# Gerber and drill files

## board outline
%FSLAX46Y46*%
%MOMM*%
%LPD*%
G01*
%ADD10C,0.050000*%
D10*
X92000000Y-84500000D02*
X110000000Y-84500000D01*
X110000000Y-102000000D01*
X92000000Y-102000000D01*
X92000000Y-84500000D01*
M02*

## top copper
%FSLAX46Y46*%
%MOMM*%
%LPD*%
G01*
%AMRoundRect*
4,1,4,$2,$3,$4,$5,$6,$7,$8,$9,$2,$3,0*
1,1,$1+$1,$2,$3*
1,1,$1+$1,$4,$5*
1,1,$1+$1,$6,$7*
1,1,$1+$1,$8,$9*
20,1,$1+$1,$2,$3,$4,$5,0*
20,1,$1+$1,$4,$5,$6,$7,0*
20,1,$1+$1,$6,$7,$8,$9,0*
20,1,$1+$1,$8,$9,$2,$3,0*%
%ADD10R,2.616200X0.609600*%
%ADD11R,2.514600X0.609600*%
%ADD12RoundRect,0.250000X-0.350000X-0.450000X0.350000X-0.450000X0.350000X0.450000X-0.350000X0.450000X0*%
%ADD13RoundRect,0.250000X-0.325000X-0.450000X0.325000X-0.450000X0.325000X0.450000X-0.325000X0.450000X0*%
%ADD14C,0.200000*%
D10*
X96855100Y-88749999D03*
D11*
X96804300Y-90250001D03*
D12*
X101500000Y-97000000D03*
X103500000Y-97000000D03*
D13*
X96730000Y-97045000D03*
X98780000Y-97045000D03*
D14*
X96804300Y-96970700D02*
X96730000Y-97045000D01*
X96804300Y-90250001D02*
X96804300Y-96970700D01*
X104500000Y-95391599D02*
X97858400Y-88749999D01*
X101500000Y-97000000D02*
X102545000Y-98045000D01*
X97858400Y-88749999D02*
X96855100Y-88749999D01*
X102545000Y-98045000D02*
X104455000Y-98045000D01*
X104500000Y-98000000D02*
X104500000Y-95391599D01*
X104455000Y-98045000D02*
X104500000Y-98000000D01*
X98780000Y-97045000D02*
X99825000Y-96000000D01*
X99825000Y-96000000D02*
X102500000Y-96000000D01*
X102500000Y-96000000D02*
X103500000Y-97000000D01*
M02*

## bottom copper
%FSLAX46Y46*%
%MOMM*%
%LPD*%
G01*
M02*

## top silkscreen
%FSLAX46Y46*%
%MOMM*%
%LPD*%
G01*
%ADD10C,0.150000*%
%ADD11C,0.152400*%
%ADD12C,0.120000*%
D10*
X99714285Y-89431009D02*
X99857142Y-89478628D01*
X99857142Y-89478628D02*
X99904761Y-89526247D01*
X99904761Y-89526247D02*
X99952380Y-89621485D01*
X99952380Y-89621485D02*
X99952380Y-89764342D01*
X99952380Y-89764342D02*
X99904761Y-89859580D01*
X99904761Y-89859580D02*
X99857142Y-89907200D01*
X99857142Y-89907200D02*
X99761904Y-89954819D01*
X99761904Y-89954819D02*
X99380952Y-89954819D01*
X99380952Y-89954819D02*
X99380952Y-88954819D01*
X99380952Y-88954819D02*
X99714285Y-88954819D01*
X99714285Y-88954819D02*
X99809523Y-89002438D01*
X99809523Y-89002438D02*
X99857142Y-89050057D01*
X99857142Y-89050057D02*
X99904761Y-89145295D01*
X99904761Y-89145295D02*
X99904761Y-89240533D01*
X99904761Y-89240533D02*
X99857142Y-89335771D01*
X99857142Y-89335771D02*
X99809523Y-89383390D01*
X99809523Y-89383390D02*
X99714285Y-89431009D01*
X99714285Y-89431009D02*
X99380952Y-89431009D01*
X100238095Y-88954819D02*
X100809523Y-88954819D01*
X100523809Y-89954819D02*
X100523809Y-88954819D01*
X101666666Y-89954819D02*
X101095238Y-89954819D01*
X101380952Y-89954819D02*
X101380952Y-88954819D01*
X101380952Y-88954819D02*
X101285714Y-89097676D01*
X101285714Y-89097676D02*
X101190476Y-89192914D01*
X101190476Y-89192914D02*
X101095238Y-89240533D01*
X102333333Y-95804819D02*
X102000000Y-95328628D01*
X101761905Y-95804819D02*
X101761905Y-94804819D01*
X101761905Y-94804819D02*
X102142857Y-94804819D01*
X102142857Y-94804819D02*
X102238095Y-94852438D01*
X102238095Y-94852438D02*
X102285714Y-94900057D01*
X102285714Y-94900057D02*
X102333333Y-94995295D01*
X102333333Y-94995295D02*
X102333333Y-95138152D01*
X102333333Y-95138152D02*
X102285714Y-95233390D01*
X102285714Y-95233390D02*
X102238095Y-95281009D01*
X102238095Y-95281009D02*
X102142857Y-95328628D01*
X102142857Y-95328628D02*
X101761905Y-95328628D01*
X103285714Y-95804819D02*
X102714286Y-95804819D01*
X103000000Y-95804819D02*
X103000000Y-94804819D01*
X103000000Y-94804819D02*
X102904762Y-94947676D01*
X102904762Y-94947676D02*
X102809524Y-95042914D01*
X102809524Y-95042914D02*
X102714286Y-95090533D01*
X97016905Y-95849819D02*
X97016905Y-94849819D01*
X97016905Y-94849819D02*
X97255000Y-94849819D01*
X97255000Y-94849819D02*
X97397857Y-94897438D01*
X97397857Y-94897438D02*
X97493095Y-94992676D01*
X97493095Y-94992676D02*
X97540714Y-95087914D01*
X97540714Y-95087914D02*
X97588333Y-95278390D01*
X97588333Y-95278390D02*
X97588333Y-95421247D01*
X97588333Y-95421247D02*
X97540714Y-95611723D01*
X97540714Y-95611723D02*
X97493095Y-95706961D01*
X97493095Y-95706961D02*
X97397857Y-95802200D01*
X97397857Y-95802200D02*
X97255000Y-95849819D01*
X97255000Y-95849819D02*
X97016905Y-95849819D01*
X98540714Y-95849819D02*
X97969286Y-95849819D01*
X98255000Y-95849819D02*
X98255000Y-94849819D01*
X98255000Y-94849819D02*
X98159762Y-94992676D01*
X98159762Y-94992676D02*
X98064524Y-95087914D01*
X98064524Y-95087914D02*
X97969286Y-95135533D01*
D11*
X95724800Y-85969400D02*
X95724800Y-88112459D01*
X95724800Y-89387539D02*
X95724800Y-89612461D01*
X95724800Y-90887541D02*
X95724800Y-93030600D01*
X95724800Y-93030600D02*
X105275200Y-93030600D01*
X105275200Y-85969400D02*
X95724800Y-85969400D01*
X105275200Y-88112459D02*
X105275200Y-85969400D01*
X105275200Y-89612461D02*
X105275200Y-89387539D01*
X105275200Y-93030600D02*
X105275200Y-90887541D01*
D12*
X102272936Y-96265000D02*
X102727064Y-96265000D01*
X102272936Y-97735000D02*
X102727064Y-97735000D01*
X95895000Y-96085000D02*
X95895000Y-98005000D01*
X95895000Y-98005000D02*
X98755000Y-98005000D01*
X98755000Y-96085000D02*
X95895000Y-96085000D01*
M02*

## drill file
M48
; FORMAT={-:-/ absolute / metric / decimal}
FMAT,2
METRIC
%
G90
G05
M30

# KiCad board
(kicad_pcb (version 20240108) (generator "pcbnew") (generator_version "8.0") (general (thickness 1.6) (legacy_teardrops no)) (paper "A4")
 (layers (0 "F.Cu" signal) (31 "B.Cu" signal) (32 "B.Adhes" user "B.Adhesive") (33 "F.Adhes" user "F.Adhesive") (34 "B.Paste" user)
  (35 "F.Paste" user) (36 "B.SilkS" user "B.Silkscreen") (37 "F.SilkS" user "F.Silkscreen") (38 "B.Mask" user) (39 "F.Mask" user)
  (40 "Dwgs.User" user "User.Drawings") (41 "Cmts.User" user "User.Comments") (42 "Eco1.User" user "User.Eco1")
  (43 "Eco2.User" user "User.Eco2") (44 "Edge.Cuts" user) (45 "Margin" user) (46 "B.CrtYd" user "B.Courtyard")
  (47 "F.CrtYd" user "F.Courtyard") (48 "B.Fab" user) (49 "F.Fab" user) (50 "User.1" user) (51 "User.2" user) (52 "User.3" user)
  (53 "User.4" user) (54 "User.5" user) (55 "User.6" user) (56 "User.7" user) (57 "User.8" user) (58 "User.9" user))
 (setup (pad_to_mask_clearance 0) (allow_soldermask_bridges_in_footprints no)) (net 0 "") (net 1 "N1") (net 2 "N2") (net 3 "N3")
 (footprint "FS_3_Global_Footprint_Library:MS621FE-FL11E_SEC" (layer "F.Cu") (at 100.5 89.5)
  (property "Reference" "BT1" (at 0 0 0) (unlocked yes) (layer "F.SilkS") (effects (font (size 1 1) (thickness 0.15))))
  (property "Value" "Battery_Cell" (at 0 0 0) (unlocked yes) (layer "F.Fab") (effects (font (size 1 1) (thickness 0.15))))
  (fp_line (start -4.7752 -3.5306) (end -4.7752 -1.387541) (stroke (width 0.1524) (type solid)) (layer "F.SilkS"))
  (fp_line (start -4.7752 -0.112461) (end -4.7752 0.112461) (stroke (width 0.1524) (type solid)) (layer "F.SilkS"))
  (fp_line (start -4.7752 1.387541) (end -4.7752 3.5306) (stroke (width 0.1524) (type solid)) (layer "F.SilkS"))
  (fp_line (start -4.7752 3.5306) (end 4.7752 3.5306) (stroke (width 0.1524) (type solid)) (layer "F.SilkS"))
  (fp_line (start 4.7752 -3.5306) (end -4.7752 -3.5306) (stroke (width 0.1524) (type solid)) (layer "F.SilkS"))
  (fp_line (start 4.7752 -1.387541) (end 4.7752 -3.5306) (stroke (width 0.1524) (type solid)) (layer "F.SilkS"))
  (fp_line (start 4.7752 0.112461) (end 4.7752 -0.112461) (stroke (width 0.1524) (type solid)) (layer "F.SilkS"))
  (fp_line (start 4.7752 3.5306) (end 4.7752 1.387541) (stroke (width 0.1524) (type solid)) (layer "F.SilkS"))
  (pad "1" smd rect (at -3.6449 -0.750001) (size 2.6162 0.6096) (layers "F.Cu" "F.Paste" "F.Mask") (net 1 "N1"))
  (pad "2" smd rect (at -3.6957 0.750001) (size 2.5146 0.6096) (layers "F.Cu" "F.Paste" "F.Mask") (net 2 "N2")))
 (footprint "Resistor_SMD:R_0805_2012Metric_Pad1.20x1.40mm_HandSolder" (layer "F.Cu") (at 102.5 97)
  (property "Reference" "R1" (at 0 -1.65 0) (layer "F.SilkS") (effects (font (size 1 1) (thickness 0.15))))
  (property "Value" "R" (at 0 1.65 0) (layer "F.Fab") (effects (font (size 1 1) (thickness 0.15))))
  (fp_line (start -0.227064 -0.735) (end 0.227064 -0.735) (stroke (width 0.12) (type solid)) (layer "F.SilkS"))
  (fp_line (start -0.227064 0.735) (end 0.227064 0.735) (stroke (width 0.12) (type solid)) (layer "F.SilkS"))
  (pad "1" smd roundrect (at -1 0) (size 1.2 1.4) (layers "F.Cu" "F.Paste" "F.Mask") (roundrect_rratio 0.208333) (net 1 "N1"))
  (pad "2" smd roundrect (at 1 0) (size 1.2 1.4) (layers "F.Cu" "F.Paste" "F.Mask") (roundrect_rratio 0.208333) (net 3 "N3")))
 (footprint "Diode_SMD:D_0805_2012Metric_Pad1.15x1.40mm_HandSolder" (layer "F.Cu") (at 97.755 97.045)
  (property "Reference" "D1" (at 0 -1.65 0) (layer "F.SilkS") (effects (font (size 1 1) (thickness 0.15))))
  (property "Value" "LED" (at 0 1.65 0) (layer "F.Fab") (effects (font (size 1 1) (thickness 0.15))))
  (fp_line (start -1.86 -0.96) (end -1.86 0.96) (stroke (width 0.12) (type solid)) (layer "F.SilkS"))
  (fp_line (start -1.86 0.96) (end 1 0.96) (stroke (width 0.12) (type solid)) (layer "F.SilkS"))
  (fp_line (start 1 -0.96) (end -1.86 -0.96) (stroke (width 0.12) (type solid)) (layer "F.SilkS"))
  (pad "1" smd roundrect (at -1.025 0) (size 1.15 1.4) (layers "F.Cu" "F.Paste" "F.Mask") (roundrect_rratio 0.217391) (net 2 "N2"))
  (pad "2" smd roundrect (at 1.025 0) (size 1.15 1.4) (layers "F.Cu" "F.Paste" "F.Mask") (roundrect_rratio 0.217391) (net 3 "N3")))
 (gr_rect (start 92 84.5) (end 110 102) (stroke (width 0.05) (type default)) (fill none) (layer "Edge.Cuts"))
 (segment (start 96.8043 96.9707) (end 96.73 97.045) (width 0.2) (layer "F.Cu") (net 2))
 (segment (start 96.8043 90.250001) (end 96.8043 96.9707) (width 0.2) (layer "F.Cu") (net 2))
 (segment (start 104.5 95.391599) (end 97.8584 88.749999) (width 0.2) (layer "F.Cu") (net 1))
 (segment (start 101.5 97) (end 102.545 98.045) (width 0.2) (layer "F.Cu") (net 1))
 (segment (start 97.8584 88.749999) (end 96.8551 88.749999) (width 0.2) (layer "F.Cu") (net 1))
 (segment (start 102.545 98.045) (end 104.455 98.045) (width 0.2) (layer "F.Cu") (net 1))
 (segment (start 104.5 98) (end 104.5 95.391599) (width 0.2) (layer "F.Cu") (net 1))
 (segment (start 104.455 98.045) (end 104.5 98) (width 0.2) (layer "F.Cu") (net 1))
 (segment (start 98.78 97.045) (end 99.825 96) (width 0.2) (layer "F.Cu") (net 3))
 (segment (start 99.825 96) (end 102.5 96) (width 0.2) (layer "F.Cu") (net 3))
 (segment (start 102.5 96) (end 103.5 97) (width 0.2) (layer "F.Cu") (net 3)))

